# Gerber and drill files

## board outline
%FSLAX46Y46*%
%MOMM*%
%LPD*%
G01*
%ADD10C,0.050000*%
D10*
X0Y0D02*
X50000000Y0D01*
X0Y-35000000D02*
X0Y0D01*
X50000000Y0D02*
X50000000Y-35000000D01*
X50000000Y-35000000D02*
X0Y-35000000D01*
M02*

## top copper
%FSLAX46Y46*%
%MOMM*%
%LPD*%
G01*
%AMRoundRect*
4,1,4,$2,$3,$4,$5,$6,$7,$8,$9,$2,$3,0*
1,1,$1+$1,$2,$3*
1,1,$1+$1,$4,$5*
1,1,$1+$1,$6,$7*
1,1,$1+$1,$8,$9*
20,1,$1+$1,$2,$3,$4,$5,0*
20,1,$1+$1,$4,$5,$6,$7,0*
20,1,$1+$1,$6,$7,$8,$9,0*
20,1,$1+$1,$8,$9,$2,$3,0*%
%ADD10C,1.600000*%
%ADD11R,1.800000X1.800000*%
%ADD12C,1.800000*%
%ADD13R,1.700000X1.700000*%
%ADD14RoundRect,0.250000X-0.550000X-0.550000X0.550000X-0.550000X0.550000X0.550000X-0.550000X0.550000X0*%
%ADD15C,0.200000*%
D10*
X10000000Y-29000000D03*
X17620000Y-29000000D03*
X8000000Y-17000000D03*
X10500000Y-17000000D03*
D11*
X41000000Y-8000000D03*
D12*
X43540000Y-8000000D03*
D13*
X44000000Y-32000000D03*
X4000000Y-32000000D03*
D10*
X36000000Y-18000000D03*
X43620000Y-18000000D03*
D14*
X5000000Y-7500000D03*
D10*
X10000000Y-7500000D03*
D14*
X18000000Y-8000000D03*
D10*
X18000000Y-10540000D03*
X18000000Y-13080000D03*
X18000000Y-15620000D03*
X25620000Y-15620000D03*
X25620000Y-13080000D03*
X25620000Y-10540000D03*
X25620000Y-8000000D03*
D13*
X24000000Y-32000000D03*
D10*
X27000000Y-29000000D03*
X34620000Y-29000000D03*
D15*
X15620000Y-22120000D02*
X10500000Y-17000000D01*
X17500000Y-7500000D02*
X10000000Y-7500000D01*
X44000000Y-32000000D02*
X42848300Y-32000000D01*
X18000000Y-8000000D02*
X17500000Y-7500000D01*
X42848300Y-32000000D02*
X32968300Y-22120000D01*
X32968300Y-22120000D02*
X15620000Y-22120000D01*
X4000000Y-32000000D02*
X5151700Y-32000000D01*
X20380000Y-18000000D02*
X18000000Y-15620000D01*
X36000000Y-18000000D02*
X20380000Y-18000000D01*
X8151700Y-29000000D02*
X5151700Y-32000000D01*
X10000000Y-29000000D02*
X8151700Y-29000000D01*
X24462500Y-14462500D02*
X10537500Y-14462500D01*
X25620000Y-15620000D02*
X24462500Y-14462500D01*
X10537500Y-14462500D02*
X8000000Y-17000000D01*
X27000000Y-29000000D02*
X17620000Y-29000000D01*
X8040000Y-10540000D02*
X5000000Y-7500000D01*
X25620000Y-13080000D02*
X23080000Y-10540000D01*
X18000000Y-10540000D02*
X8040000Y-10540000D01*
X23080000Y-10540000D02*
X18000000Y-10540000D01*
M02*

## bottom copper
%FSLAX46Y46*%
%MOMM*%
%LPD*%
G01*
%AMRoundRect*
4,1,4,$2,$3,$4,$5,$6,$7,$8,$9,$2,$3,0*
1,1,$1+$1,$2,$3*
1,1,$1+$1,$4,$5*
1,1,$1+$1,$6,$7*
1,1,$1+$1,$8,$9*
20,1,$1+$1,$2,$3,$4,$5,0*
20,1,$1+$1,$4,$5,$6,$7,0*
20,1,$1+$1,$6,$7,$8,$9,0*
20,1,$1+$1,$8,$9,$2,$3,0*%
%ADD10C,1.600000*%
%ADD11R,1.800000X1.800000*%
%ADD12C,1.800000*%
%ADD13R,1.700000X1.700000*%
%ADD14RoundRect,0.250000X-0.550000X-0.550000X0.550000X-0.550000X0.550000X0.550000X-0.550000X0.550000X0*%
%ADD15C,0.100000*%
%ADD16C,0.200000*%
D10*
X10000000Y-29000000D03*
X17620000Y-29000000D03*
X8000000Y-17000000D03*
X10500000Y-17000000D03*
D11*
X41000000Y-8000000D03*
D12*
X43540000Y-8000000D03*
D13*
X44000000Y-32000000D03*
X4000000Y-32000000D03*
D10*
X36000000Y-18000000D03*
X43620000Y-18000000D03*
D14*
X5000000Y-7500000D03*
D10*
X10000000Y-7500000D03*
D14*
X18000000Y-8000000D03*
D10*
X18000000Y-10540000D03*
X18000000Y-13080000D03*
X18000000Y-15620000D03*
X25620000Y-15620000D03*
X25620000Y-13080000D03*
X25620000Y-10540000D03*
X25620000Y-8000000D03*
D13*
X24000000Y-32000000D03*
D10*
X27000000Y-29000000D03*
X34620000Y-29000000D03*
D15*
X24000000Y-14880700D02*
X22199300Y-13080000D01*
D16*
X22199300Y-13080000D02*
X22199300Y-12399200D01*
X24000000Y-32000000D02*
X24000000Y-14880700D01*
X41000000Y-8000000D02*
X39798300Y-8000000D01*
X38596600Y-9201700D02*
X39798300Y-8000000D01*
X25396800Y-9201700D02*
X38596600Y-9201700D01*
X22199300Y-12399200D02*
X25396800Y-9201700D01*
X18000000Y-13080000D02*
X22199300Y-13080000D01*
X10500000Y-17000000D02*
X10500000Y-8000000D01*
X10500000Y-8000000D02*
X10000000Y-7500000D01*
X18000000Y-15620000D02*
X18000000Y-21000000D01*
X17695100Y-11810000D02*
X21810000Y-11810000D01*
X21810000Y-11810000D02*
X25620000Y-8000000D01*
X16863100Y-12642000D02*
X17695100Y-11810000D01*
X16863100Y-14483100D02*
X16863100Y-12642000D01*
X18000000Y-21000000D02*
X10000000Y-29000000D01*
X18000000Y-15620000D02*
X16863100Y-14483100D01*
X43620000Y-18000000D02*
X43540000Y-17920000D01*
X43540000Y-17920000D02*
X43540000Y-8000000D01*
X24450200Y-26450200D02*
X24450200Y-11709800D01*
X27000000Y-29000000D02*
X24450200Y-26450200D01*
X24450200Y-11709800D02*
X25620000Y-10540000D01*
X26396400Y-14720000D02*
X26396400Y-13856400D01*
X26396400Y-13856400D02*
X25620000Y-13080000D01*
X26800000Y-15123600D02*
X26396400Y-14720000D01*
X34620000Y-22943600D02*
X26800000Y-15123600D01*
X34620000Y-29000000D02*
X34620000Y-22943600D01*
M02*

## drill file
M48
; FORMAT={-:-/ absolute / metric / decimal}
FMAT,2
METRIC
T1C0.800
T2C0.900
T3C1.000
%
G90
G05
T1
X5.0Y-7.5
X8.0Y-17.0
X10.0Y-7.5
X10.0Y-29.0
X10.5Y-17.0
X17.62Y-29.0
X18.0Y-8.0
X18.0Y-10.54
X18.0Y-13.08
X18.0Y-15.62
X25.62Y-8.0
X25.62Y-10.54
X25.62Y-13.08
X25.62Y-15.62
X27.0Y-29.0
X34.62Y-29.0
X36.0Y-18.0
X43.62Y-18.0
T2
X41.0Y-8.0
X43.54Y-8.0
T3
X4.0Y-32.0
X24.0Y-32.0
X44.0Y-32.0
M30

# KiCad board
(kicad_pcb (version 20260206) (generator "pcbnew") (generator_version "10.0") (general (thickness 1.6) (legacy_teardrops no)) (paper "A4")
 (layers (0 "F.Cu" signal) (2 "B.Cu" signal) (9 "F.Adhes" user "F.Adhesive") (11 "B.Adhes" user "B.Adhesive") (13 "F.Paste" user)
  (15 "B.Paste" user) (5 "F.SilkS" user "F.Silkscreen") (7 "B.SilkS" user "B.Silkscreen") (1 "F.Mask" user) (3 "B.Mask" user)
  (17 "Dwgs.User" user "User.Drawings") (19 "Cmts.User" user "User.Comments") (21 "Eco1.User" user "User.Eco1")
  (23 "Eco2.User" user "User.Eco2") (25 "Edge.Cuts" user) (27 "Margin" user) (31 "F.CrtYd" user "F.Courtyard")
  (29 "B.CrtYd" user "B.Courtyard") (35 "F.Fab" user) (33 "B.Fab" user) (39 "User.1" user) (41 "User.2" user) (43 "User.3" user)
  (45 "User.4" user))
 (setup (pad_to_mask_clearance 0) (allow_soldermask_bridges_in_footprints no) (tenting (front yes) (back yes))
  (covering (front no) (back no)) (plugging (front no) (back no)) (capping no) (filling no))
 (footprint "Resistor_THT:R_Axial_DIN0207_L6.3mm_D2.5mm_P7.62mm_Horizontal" (layer "F.Cu") (at 10 29)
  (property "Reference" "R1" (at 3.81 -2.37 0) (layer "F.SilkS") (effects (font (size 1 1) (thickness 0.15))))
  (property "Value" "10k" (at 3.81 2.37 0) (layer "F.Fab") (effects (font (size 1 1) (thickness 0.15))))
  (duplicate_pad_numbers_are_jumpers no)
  (pad "1" thru_hole circle (at 0 0) (size 1.6 1.6) (drill 0.8) (layers "*.Cu" "*.Mask") (remove_unused_layers no) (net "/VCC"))
  (pad "2" thru_hole circle (at 7.62 0) (size 1.6 1.6) (drill 0.8) (layers "*.Cu" "*.Mask") (remove_unused_layers no) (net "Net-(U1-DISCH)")))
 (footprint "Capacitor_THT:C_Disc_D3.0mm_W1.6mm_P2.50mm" (layer "F.Cu") (at 8 17)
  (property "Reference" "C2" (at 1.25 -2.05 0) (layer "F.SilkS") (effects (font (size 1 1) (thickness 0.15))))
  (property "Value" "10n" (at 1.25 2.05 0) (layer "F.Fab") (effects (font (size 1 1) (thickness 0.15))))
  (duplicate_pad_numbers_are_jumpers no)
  (pad "1" thru_hole circle (at 0 0) (size 1.6 1.6) (drill 0.8) (layers "*.Cu" "*.Mask") (remove_unused_layers no) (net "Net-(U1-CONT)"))
  (pad "2" thru_hole circle (at 2.5 0) (size 1.6 1.6) (drill 0.8) (layers "*.Cu" "*.Mask") (remove_unused_layers no) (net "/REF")))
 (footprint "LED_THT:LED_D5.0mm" (layer "F.Cu") (at 41 8)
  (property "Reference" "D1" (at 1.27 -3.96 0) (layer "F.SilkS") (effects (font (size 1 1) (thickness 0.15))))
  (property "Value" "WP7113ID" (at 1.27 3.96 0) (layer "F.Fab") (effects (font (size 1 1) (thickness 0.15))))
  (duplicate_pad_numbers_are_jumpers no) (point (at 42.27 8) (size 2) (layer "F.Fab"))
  (pad "1" thru_hole rect (at 0 0) (size 1.8 1.8) (drill 0.9) (layers "*.Cu" "*.Mask") (remove_unused_layers no) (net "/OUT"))
  (pad "2" thru_hole circle (at 2.54 0) (size 1.8 1.8) (drill 0.9) (layers "*.Cu" "*.Mask") (remove_unused_layers no) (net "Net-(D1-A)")))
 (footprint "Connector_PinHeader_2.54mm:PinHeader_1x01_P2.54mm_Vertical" (layer "F.Cu") (at 44 32)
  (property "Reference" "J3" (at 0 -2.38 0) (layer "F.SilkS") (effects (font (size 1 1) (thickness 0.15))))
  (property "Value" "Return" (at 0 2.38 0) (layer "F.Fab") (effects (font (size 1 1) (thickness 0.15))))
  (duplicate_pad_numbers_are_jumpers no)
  (pad "1" thru_hole rect (at 0 0) (size 1.7 1.7) (drill 1) (layers "*.Cu" "*.Mask") (remove_unused_layers no) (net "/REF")))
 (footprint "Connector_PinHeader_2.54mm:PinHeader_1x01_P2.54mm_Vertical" (layer "F.Cu") (at 4 32)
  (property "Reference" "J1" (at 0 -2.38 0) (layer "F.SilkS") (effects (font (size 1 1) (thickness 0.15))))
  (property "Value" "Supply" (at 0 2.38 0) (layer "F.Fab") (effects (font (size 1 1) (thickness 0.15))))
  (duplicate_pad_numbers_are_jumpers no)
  (pad "1" thru_hole rect (at 0 0) (size 1.7 1.7) (drill 1) (layers "*.Cu" "*.Mask") (remove_unused_layers no) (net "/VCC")))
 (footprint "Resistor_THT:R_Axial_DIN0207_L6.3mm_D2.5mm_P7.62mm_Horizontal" (layer "F.Cu") (at 36 18)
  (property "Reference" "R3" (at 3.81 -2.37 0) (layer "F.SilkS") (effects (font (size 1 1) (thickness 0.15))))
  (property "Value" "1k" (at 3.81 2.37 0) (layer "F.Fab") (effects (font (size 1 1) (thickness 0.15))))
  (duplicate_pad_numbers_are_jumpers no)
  (pad "1" thru_hole circle (at 0 0) (size 1.6 1.6) (drill 0.8) (layers "*.Cu" "*.Mask") (remove_unused_layers no) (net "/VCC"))
  (pad "2" thru_hole circle (at 7.62 0) (size 1.6 1.6) (drill 0.8) (layers "*.Cu" "*.Mask") (remove_unused_layers no) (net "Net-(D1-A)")))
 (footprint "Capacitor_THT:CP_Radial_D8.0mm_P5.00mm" (layer "F.Cu") (at 5 7.5)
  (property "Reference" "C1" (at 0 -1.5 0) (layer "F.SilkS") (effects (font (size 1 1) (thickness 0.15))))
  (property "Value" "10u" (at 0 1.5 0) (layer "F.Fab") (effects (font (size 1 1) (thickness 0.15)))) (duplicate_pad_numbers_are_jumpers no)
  (pad "1" thru_hole roundrect (at 0 0) (size 1.6 1.6) (drill 0.8) (layers "*.Cu" "*.Mask") (remove_unused_layers no)
   (roundrect_rratio 0.15625) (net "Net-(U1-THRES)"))
  (pad "2" thru_hole circle (at 5 0) (size 1.6 1.6) (drill 0.8) (layers "*.Cu" "*.Mask") (remove_unused_layers no) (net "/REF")))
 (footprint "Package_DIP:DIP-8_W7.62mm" (layer "F.Cu") (at 18 8)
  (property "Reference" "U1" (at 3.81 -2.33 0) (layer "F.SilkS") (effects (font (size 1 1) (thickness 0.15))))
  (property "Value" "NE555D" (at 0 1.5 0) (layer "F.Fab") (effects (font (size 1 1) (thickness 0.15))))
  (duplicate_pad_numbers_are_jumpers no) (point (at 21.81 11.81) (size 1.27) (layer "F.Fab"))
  (pad "1" thru_hole roundrect (at 0 0) (size 1.6 1.6) (drill 0.8) (layers "*.Cu" "*.Mask") (remove_unused_layers no)
   (roundrect_rratio 0.15625) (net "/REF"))
  (pad "2" thru_hole circle (at 0 2.54) (size 1.6 1.6) (drill 0.8) (layers "*.Cu" "*.Mask") (remove_unused_layers no) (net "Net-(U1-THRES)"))
  (pad "3" thru_hole circle (at 0 5.08) (size 1.6 1.6) (drill 0.8) (layers "*.Cu" "*.Mask") (remove_unused_layers no) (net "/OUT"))
  (pad "4" thru_hole circle (at 0 7.62) (size 1.6 1.6) (drill 0.8) (layers "*.Cu" "*.Mask") (remove_unused_layers no) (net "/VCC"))
  (pad "5" thru_hole circle (at 7.62 7.62) (size 1.6 1.6) (drill 0.8) (layers "*.Cu" "*.Mask") (remove_unused_layers no)
   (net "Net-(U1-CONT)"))
  (pad "6" thru_hole circle (at 7.62 5.08) (size 1.6 1.6) (drill 0.8) (layers "*.Cu" "*.Mask") (remove_unused_layers no)
   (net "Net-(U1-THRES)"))
  (pad "7" thru_hole circle (at 7.62 2.54) (size 1.6 1.6) (drill 0.8) (layers "*.Cu" "*.Mask") (remove_unused_layers no)
   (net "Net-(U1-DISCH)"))
  (pad "8" thru_hole circle (at 7.62 0) (size 1.6 1.6) (drill 0.8) (layers "*.Cu" "*.Mask") (remove_unused_layers no) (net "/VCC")))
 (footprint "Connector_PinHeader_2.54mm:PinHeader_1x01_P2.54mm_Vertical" (layer "F.Cu") (at 24 32)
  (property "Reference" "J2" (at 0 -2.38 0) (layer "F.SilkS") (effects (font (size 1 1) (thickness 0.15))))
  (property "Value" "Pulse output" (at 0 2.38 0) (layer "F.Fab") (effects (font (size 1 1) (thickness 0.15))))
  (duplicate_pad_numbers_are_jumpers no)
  (pad "1" thru_hole rect (at 0 0) (size 1.7 1.7) (drill 1) (layers "*.Cu" "*.Mask") (remove_unused_layers no) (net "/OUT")))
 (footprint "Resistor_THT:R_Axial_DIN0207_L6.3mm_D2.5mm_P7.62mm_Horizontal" (layer "F.Cu") (at 27 29)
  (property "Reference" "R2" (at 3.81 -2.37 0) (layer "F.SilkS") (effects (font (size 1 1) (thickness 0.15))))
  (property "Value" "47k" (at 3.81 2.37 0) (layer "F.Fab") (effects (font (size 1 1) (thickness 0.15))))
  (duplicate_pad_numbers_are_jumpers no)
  (pad "1" thru_hole circle (at 0 0) (size 1.6 1.6) (drill 0.8) (layers "*.Cu" "*.Mask") (remove_unused_layers no) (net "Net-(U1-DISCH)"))
  (pad "2" thru_hole circle (at 7.62 0) (size 1.6 1.6) (drill 0.8) (layers "*.Cu" "*.Mask") (remove_unused_layers no) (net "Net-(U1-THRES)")))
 (gr_line (start 0 0) (end 50 0) (stroke (width 0.05) (type default)) (layer "Edge.Cuts"))
 (gr_line (start 0 35) (end 0 0) (stroke (width 0.05) (type default)) (layer "Edge.Cuts"))
 (gr_line (start 50 0) (end 50 35) (stroke (width 0.05) (type default)) (layer "Edge.Cuts"))
 (gr_line (start 50 35) (end 0 35) (stroke (width 0.05) (type default)) (layer "Edge.Cuts"))
 (segment (start 24 14.8807) (end 22.1993 13.08) (width 0.100000) (layer "B.Cu") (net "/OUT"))
 (segment (start 22.1993 13.08) (end 22.1993 12.3992) (width 0.2) (layer "B.Cu") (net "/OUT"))
 (segment (start 24 32) (end 24 14.8807) (width 0.2) (layer "B.Cu") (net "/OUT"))
 (segment (start 41 8) (end 39.7983 8) (width 0.2) (layer "B.Cu") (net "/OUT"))
 (segment (start 38.5966 9.2017) (end 39.7983 8) (width 0.2) (layer "B.Cu") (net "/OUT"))
 (segment (start 25.3968 9.2017) (end 38.5966 9.2017) (width 0.2) (layer "B.Cu") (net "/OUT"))
 (segment (start 22.1993 12.3992) (end 25.3968 9.2017) (width 0.2) (layer "B.Cu") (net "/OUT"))
 (segment (start 18 13.08) (end 22.1993 13.08) (width 0.2) (layer "B.Cu") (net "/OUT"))
 (segment (start 15.62 22.12) (end 10.5 17) (width 0.2) (layer "F.Cu") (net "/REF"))
 (segment (start 17.5 7.5) (end 10 7.5) (width 0.2) (layer "F.Cu") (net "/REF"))
 (segment (start 44 32) (end 42.8483 32) (width 0.2) (layer "F.Cu") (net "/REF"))
 (segment (start 18 8) (end 17.5 7.5) (width 0.2) (layer "F.Cu") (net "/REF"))
 (segment (start 42.8483 32) (end 32.9683 22.12) (width 0.2) (layer "F.Cu") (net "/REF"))
 (segment (start 32.9683 22.12) (end 15.62 22.12) (width 0.2) (layer "F.Cu") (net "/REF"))
 (segment (start 10.5 17) (end 10.5 8) (width 0.2) (layer "B.Cu") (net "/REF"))
 (segment (start 10.5 8) (end 10 7.5) (width 0.2) (layer "B.Cu") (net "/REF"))
 (segment (start 4 32) (end 5.1517 32) (width 0.2) (layer "F.Cu") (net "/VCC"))
 (segment (start 20.38 18) (end 18 15.62) (width 0.2) (layer "F.Cu") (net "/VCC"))
 (segment (start 36 18) (end 20.38 18) (width 0.2) (layer "F.Cu") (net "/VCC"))
 (segment (start 8.1517 29) (end 5.1517 32) (width 0.2) (layer "F.Cu") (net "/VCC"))
 (segment (start 10 29) (end 8.1517 29) (width 0.2) (layer "F.Cu") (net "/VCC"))
 (segment (start 18 15.62) (end 18 21) (width 0.2) (layer "B.Cu") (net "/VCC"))
 (segment (start 17.6951 11.81) (end 21.81 11.81) (width 0.2) (layer "B.Cu") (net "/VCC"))
 (segment (start 21.81 11.81) (end 25.62 8) (width 0.2) (layer "B.Cu") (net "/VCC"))
 (segment (start 16.8631 12.642) (end 17.6951 11.81) (width 0.2) (layer "B.Cu") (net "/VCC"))
 (segment (start 16.8631 14.4831) (end 16.8631 12.642) (width 0.2) (layer "B.Cu") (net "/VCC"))
 (segment (start 18 21) (end 10 29) (width 0.2) (layer "B.Cu") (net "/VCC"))
 (segment (start 18 15.62) (end 16.8631 14.4831) (width 0.2) (layer "B.Cu") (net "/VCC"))
 (segment (start 43.62 18) (end 43.54 17.92) (width 0.2) (layer "B.Cu") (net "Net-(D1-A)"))
 (segment (start 43.54 17.92) (end 43.54 8) (width 0.2) (layer "B.Cu") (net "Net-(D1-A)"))
 (segment (start 24.4625 14.4625) (end 10.5375 14.4625) (width 0.2) (layer "F.Cu") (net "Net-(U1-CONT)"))
 (segment (start 25.62 15.62) (end 24.4625 14.4625) (width 0.2) (layer "F.Cu") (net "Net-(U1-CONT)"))
 (segment (start 10.5375 14.4625) (end 8 17) (width 0.2) (layer "F.Cu") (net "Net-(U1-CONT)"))
 (segment (start 27 29) (end 17.62 29) (width 0.2) (layer "F.Cu") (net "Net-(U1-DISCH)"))
 (segment (start 24.4502 26.4502) (end 24.4502 11.7098) (width 0.2) (layer "B.Cu") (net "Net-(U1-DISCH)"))
 (segment (start 27 29) (end 24.4502 26.4502) (width 0.2) (layer "B.Cu") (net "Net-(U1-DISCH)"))
 (segment (start 24.4502 11.7098) (end 25.62 10.54) (width 0.2) (layer "B.Cu") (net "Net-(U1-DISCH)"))
 (segment (start 8.04 10.54) (end 5 7.5) (width 0.2) (layer "F.Cu") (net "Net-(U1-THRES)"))
 (segment (start 25.62 13.08) (end 23.08 10.54) (width 0.2) (layer "F.Cu") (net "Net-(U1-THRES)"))
 (segment (start 18 10.54) (end 8.04 10.54) (width 0.2) (layer "F.Cu") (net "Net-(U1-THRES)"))
 (segment (start 23.08 10.54) (end 18 10.54) (width 0.2) (layer "F.Cu") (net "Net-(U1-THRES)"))
 (segment (start 26.3964 14.72) (end 26.3964 13.8564) (width 0.2) (layer "B.Cu") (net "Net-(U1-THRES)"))
 (segment (start 26.3964 13.8564) (end 25.62 13.08) (width 0.2) (layer "B.Cu") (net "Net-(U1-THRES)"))
 (segment (start 26.8 15.1236) (end 26.3964 14.72) (width 0.2) (layer "B.Cu") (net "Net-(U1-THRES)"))
 (segment (start 34.62 22.9436) (end 26.8 15.1236) (width 0.2) (layer "B.Cu") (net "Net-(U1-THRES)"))
 (segment (start 34.62 29) (end 34.62 22.9436) (width 0.2) (layer "B.Cu") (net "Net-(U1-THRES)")))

